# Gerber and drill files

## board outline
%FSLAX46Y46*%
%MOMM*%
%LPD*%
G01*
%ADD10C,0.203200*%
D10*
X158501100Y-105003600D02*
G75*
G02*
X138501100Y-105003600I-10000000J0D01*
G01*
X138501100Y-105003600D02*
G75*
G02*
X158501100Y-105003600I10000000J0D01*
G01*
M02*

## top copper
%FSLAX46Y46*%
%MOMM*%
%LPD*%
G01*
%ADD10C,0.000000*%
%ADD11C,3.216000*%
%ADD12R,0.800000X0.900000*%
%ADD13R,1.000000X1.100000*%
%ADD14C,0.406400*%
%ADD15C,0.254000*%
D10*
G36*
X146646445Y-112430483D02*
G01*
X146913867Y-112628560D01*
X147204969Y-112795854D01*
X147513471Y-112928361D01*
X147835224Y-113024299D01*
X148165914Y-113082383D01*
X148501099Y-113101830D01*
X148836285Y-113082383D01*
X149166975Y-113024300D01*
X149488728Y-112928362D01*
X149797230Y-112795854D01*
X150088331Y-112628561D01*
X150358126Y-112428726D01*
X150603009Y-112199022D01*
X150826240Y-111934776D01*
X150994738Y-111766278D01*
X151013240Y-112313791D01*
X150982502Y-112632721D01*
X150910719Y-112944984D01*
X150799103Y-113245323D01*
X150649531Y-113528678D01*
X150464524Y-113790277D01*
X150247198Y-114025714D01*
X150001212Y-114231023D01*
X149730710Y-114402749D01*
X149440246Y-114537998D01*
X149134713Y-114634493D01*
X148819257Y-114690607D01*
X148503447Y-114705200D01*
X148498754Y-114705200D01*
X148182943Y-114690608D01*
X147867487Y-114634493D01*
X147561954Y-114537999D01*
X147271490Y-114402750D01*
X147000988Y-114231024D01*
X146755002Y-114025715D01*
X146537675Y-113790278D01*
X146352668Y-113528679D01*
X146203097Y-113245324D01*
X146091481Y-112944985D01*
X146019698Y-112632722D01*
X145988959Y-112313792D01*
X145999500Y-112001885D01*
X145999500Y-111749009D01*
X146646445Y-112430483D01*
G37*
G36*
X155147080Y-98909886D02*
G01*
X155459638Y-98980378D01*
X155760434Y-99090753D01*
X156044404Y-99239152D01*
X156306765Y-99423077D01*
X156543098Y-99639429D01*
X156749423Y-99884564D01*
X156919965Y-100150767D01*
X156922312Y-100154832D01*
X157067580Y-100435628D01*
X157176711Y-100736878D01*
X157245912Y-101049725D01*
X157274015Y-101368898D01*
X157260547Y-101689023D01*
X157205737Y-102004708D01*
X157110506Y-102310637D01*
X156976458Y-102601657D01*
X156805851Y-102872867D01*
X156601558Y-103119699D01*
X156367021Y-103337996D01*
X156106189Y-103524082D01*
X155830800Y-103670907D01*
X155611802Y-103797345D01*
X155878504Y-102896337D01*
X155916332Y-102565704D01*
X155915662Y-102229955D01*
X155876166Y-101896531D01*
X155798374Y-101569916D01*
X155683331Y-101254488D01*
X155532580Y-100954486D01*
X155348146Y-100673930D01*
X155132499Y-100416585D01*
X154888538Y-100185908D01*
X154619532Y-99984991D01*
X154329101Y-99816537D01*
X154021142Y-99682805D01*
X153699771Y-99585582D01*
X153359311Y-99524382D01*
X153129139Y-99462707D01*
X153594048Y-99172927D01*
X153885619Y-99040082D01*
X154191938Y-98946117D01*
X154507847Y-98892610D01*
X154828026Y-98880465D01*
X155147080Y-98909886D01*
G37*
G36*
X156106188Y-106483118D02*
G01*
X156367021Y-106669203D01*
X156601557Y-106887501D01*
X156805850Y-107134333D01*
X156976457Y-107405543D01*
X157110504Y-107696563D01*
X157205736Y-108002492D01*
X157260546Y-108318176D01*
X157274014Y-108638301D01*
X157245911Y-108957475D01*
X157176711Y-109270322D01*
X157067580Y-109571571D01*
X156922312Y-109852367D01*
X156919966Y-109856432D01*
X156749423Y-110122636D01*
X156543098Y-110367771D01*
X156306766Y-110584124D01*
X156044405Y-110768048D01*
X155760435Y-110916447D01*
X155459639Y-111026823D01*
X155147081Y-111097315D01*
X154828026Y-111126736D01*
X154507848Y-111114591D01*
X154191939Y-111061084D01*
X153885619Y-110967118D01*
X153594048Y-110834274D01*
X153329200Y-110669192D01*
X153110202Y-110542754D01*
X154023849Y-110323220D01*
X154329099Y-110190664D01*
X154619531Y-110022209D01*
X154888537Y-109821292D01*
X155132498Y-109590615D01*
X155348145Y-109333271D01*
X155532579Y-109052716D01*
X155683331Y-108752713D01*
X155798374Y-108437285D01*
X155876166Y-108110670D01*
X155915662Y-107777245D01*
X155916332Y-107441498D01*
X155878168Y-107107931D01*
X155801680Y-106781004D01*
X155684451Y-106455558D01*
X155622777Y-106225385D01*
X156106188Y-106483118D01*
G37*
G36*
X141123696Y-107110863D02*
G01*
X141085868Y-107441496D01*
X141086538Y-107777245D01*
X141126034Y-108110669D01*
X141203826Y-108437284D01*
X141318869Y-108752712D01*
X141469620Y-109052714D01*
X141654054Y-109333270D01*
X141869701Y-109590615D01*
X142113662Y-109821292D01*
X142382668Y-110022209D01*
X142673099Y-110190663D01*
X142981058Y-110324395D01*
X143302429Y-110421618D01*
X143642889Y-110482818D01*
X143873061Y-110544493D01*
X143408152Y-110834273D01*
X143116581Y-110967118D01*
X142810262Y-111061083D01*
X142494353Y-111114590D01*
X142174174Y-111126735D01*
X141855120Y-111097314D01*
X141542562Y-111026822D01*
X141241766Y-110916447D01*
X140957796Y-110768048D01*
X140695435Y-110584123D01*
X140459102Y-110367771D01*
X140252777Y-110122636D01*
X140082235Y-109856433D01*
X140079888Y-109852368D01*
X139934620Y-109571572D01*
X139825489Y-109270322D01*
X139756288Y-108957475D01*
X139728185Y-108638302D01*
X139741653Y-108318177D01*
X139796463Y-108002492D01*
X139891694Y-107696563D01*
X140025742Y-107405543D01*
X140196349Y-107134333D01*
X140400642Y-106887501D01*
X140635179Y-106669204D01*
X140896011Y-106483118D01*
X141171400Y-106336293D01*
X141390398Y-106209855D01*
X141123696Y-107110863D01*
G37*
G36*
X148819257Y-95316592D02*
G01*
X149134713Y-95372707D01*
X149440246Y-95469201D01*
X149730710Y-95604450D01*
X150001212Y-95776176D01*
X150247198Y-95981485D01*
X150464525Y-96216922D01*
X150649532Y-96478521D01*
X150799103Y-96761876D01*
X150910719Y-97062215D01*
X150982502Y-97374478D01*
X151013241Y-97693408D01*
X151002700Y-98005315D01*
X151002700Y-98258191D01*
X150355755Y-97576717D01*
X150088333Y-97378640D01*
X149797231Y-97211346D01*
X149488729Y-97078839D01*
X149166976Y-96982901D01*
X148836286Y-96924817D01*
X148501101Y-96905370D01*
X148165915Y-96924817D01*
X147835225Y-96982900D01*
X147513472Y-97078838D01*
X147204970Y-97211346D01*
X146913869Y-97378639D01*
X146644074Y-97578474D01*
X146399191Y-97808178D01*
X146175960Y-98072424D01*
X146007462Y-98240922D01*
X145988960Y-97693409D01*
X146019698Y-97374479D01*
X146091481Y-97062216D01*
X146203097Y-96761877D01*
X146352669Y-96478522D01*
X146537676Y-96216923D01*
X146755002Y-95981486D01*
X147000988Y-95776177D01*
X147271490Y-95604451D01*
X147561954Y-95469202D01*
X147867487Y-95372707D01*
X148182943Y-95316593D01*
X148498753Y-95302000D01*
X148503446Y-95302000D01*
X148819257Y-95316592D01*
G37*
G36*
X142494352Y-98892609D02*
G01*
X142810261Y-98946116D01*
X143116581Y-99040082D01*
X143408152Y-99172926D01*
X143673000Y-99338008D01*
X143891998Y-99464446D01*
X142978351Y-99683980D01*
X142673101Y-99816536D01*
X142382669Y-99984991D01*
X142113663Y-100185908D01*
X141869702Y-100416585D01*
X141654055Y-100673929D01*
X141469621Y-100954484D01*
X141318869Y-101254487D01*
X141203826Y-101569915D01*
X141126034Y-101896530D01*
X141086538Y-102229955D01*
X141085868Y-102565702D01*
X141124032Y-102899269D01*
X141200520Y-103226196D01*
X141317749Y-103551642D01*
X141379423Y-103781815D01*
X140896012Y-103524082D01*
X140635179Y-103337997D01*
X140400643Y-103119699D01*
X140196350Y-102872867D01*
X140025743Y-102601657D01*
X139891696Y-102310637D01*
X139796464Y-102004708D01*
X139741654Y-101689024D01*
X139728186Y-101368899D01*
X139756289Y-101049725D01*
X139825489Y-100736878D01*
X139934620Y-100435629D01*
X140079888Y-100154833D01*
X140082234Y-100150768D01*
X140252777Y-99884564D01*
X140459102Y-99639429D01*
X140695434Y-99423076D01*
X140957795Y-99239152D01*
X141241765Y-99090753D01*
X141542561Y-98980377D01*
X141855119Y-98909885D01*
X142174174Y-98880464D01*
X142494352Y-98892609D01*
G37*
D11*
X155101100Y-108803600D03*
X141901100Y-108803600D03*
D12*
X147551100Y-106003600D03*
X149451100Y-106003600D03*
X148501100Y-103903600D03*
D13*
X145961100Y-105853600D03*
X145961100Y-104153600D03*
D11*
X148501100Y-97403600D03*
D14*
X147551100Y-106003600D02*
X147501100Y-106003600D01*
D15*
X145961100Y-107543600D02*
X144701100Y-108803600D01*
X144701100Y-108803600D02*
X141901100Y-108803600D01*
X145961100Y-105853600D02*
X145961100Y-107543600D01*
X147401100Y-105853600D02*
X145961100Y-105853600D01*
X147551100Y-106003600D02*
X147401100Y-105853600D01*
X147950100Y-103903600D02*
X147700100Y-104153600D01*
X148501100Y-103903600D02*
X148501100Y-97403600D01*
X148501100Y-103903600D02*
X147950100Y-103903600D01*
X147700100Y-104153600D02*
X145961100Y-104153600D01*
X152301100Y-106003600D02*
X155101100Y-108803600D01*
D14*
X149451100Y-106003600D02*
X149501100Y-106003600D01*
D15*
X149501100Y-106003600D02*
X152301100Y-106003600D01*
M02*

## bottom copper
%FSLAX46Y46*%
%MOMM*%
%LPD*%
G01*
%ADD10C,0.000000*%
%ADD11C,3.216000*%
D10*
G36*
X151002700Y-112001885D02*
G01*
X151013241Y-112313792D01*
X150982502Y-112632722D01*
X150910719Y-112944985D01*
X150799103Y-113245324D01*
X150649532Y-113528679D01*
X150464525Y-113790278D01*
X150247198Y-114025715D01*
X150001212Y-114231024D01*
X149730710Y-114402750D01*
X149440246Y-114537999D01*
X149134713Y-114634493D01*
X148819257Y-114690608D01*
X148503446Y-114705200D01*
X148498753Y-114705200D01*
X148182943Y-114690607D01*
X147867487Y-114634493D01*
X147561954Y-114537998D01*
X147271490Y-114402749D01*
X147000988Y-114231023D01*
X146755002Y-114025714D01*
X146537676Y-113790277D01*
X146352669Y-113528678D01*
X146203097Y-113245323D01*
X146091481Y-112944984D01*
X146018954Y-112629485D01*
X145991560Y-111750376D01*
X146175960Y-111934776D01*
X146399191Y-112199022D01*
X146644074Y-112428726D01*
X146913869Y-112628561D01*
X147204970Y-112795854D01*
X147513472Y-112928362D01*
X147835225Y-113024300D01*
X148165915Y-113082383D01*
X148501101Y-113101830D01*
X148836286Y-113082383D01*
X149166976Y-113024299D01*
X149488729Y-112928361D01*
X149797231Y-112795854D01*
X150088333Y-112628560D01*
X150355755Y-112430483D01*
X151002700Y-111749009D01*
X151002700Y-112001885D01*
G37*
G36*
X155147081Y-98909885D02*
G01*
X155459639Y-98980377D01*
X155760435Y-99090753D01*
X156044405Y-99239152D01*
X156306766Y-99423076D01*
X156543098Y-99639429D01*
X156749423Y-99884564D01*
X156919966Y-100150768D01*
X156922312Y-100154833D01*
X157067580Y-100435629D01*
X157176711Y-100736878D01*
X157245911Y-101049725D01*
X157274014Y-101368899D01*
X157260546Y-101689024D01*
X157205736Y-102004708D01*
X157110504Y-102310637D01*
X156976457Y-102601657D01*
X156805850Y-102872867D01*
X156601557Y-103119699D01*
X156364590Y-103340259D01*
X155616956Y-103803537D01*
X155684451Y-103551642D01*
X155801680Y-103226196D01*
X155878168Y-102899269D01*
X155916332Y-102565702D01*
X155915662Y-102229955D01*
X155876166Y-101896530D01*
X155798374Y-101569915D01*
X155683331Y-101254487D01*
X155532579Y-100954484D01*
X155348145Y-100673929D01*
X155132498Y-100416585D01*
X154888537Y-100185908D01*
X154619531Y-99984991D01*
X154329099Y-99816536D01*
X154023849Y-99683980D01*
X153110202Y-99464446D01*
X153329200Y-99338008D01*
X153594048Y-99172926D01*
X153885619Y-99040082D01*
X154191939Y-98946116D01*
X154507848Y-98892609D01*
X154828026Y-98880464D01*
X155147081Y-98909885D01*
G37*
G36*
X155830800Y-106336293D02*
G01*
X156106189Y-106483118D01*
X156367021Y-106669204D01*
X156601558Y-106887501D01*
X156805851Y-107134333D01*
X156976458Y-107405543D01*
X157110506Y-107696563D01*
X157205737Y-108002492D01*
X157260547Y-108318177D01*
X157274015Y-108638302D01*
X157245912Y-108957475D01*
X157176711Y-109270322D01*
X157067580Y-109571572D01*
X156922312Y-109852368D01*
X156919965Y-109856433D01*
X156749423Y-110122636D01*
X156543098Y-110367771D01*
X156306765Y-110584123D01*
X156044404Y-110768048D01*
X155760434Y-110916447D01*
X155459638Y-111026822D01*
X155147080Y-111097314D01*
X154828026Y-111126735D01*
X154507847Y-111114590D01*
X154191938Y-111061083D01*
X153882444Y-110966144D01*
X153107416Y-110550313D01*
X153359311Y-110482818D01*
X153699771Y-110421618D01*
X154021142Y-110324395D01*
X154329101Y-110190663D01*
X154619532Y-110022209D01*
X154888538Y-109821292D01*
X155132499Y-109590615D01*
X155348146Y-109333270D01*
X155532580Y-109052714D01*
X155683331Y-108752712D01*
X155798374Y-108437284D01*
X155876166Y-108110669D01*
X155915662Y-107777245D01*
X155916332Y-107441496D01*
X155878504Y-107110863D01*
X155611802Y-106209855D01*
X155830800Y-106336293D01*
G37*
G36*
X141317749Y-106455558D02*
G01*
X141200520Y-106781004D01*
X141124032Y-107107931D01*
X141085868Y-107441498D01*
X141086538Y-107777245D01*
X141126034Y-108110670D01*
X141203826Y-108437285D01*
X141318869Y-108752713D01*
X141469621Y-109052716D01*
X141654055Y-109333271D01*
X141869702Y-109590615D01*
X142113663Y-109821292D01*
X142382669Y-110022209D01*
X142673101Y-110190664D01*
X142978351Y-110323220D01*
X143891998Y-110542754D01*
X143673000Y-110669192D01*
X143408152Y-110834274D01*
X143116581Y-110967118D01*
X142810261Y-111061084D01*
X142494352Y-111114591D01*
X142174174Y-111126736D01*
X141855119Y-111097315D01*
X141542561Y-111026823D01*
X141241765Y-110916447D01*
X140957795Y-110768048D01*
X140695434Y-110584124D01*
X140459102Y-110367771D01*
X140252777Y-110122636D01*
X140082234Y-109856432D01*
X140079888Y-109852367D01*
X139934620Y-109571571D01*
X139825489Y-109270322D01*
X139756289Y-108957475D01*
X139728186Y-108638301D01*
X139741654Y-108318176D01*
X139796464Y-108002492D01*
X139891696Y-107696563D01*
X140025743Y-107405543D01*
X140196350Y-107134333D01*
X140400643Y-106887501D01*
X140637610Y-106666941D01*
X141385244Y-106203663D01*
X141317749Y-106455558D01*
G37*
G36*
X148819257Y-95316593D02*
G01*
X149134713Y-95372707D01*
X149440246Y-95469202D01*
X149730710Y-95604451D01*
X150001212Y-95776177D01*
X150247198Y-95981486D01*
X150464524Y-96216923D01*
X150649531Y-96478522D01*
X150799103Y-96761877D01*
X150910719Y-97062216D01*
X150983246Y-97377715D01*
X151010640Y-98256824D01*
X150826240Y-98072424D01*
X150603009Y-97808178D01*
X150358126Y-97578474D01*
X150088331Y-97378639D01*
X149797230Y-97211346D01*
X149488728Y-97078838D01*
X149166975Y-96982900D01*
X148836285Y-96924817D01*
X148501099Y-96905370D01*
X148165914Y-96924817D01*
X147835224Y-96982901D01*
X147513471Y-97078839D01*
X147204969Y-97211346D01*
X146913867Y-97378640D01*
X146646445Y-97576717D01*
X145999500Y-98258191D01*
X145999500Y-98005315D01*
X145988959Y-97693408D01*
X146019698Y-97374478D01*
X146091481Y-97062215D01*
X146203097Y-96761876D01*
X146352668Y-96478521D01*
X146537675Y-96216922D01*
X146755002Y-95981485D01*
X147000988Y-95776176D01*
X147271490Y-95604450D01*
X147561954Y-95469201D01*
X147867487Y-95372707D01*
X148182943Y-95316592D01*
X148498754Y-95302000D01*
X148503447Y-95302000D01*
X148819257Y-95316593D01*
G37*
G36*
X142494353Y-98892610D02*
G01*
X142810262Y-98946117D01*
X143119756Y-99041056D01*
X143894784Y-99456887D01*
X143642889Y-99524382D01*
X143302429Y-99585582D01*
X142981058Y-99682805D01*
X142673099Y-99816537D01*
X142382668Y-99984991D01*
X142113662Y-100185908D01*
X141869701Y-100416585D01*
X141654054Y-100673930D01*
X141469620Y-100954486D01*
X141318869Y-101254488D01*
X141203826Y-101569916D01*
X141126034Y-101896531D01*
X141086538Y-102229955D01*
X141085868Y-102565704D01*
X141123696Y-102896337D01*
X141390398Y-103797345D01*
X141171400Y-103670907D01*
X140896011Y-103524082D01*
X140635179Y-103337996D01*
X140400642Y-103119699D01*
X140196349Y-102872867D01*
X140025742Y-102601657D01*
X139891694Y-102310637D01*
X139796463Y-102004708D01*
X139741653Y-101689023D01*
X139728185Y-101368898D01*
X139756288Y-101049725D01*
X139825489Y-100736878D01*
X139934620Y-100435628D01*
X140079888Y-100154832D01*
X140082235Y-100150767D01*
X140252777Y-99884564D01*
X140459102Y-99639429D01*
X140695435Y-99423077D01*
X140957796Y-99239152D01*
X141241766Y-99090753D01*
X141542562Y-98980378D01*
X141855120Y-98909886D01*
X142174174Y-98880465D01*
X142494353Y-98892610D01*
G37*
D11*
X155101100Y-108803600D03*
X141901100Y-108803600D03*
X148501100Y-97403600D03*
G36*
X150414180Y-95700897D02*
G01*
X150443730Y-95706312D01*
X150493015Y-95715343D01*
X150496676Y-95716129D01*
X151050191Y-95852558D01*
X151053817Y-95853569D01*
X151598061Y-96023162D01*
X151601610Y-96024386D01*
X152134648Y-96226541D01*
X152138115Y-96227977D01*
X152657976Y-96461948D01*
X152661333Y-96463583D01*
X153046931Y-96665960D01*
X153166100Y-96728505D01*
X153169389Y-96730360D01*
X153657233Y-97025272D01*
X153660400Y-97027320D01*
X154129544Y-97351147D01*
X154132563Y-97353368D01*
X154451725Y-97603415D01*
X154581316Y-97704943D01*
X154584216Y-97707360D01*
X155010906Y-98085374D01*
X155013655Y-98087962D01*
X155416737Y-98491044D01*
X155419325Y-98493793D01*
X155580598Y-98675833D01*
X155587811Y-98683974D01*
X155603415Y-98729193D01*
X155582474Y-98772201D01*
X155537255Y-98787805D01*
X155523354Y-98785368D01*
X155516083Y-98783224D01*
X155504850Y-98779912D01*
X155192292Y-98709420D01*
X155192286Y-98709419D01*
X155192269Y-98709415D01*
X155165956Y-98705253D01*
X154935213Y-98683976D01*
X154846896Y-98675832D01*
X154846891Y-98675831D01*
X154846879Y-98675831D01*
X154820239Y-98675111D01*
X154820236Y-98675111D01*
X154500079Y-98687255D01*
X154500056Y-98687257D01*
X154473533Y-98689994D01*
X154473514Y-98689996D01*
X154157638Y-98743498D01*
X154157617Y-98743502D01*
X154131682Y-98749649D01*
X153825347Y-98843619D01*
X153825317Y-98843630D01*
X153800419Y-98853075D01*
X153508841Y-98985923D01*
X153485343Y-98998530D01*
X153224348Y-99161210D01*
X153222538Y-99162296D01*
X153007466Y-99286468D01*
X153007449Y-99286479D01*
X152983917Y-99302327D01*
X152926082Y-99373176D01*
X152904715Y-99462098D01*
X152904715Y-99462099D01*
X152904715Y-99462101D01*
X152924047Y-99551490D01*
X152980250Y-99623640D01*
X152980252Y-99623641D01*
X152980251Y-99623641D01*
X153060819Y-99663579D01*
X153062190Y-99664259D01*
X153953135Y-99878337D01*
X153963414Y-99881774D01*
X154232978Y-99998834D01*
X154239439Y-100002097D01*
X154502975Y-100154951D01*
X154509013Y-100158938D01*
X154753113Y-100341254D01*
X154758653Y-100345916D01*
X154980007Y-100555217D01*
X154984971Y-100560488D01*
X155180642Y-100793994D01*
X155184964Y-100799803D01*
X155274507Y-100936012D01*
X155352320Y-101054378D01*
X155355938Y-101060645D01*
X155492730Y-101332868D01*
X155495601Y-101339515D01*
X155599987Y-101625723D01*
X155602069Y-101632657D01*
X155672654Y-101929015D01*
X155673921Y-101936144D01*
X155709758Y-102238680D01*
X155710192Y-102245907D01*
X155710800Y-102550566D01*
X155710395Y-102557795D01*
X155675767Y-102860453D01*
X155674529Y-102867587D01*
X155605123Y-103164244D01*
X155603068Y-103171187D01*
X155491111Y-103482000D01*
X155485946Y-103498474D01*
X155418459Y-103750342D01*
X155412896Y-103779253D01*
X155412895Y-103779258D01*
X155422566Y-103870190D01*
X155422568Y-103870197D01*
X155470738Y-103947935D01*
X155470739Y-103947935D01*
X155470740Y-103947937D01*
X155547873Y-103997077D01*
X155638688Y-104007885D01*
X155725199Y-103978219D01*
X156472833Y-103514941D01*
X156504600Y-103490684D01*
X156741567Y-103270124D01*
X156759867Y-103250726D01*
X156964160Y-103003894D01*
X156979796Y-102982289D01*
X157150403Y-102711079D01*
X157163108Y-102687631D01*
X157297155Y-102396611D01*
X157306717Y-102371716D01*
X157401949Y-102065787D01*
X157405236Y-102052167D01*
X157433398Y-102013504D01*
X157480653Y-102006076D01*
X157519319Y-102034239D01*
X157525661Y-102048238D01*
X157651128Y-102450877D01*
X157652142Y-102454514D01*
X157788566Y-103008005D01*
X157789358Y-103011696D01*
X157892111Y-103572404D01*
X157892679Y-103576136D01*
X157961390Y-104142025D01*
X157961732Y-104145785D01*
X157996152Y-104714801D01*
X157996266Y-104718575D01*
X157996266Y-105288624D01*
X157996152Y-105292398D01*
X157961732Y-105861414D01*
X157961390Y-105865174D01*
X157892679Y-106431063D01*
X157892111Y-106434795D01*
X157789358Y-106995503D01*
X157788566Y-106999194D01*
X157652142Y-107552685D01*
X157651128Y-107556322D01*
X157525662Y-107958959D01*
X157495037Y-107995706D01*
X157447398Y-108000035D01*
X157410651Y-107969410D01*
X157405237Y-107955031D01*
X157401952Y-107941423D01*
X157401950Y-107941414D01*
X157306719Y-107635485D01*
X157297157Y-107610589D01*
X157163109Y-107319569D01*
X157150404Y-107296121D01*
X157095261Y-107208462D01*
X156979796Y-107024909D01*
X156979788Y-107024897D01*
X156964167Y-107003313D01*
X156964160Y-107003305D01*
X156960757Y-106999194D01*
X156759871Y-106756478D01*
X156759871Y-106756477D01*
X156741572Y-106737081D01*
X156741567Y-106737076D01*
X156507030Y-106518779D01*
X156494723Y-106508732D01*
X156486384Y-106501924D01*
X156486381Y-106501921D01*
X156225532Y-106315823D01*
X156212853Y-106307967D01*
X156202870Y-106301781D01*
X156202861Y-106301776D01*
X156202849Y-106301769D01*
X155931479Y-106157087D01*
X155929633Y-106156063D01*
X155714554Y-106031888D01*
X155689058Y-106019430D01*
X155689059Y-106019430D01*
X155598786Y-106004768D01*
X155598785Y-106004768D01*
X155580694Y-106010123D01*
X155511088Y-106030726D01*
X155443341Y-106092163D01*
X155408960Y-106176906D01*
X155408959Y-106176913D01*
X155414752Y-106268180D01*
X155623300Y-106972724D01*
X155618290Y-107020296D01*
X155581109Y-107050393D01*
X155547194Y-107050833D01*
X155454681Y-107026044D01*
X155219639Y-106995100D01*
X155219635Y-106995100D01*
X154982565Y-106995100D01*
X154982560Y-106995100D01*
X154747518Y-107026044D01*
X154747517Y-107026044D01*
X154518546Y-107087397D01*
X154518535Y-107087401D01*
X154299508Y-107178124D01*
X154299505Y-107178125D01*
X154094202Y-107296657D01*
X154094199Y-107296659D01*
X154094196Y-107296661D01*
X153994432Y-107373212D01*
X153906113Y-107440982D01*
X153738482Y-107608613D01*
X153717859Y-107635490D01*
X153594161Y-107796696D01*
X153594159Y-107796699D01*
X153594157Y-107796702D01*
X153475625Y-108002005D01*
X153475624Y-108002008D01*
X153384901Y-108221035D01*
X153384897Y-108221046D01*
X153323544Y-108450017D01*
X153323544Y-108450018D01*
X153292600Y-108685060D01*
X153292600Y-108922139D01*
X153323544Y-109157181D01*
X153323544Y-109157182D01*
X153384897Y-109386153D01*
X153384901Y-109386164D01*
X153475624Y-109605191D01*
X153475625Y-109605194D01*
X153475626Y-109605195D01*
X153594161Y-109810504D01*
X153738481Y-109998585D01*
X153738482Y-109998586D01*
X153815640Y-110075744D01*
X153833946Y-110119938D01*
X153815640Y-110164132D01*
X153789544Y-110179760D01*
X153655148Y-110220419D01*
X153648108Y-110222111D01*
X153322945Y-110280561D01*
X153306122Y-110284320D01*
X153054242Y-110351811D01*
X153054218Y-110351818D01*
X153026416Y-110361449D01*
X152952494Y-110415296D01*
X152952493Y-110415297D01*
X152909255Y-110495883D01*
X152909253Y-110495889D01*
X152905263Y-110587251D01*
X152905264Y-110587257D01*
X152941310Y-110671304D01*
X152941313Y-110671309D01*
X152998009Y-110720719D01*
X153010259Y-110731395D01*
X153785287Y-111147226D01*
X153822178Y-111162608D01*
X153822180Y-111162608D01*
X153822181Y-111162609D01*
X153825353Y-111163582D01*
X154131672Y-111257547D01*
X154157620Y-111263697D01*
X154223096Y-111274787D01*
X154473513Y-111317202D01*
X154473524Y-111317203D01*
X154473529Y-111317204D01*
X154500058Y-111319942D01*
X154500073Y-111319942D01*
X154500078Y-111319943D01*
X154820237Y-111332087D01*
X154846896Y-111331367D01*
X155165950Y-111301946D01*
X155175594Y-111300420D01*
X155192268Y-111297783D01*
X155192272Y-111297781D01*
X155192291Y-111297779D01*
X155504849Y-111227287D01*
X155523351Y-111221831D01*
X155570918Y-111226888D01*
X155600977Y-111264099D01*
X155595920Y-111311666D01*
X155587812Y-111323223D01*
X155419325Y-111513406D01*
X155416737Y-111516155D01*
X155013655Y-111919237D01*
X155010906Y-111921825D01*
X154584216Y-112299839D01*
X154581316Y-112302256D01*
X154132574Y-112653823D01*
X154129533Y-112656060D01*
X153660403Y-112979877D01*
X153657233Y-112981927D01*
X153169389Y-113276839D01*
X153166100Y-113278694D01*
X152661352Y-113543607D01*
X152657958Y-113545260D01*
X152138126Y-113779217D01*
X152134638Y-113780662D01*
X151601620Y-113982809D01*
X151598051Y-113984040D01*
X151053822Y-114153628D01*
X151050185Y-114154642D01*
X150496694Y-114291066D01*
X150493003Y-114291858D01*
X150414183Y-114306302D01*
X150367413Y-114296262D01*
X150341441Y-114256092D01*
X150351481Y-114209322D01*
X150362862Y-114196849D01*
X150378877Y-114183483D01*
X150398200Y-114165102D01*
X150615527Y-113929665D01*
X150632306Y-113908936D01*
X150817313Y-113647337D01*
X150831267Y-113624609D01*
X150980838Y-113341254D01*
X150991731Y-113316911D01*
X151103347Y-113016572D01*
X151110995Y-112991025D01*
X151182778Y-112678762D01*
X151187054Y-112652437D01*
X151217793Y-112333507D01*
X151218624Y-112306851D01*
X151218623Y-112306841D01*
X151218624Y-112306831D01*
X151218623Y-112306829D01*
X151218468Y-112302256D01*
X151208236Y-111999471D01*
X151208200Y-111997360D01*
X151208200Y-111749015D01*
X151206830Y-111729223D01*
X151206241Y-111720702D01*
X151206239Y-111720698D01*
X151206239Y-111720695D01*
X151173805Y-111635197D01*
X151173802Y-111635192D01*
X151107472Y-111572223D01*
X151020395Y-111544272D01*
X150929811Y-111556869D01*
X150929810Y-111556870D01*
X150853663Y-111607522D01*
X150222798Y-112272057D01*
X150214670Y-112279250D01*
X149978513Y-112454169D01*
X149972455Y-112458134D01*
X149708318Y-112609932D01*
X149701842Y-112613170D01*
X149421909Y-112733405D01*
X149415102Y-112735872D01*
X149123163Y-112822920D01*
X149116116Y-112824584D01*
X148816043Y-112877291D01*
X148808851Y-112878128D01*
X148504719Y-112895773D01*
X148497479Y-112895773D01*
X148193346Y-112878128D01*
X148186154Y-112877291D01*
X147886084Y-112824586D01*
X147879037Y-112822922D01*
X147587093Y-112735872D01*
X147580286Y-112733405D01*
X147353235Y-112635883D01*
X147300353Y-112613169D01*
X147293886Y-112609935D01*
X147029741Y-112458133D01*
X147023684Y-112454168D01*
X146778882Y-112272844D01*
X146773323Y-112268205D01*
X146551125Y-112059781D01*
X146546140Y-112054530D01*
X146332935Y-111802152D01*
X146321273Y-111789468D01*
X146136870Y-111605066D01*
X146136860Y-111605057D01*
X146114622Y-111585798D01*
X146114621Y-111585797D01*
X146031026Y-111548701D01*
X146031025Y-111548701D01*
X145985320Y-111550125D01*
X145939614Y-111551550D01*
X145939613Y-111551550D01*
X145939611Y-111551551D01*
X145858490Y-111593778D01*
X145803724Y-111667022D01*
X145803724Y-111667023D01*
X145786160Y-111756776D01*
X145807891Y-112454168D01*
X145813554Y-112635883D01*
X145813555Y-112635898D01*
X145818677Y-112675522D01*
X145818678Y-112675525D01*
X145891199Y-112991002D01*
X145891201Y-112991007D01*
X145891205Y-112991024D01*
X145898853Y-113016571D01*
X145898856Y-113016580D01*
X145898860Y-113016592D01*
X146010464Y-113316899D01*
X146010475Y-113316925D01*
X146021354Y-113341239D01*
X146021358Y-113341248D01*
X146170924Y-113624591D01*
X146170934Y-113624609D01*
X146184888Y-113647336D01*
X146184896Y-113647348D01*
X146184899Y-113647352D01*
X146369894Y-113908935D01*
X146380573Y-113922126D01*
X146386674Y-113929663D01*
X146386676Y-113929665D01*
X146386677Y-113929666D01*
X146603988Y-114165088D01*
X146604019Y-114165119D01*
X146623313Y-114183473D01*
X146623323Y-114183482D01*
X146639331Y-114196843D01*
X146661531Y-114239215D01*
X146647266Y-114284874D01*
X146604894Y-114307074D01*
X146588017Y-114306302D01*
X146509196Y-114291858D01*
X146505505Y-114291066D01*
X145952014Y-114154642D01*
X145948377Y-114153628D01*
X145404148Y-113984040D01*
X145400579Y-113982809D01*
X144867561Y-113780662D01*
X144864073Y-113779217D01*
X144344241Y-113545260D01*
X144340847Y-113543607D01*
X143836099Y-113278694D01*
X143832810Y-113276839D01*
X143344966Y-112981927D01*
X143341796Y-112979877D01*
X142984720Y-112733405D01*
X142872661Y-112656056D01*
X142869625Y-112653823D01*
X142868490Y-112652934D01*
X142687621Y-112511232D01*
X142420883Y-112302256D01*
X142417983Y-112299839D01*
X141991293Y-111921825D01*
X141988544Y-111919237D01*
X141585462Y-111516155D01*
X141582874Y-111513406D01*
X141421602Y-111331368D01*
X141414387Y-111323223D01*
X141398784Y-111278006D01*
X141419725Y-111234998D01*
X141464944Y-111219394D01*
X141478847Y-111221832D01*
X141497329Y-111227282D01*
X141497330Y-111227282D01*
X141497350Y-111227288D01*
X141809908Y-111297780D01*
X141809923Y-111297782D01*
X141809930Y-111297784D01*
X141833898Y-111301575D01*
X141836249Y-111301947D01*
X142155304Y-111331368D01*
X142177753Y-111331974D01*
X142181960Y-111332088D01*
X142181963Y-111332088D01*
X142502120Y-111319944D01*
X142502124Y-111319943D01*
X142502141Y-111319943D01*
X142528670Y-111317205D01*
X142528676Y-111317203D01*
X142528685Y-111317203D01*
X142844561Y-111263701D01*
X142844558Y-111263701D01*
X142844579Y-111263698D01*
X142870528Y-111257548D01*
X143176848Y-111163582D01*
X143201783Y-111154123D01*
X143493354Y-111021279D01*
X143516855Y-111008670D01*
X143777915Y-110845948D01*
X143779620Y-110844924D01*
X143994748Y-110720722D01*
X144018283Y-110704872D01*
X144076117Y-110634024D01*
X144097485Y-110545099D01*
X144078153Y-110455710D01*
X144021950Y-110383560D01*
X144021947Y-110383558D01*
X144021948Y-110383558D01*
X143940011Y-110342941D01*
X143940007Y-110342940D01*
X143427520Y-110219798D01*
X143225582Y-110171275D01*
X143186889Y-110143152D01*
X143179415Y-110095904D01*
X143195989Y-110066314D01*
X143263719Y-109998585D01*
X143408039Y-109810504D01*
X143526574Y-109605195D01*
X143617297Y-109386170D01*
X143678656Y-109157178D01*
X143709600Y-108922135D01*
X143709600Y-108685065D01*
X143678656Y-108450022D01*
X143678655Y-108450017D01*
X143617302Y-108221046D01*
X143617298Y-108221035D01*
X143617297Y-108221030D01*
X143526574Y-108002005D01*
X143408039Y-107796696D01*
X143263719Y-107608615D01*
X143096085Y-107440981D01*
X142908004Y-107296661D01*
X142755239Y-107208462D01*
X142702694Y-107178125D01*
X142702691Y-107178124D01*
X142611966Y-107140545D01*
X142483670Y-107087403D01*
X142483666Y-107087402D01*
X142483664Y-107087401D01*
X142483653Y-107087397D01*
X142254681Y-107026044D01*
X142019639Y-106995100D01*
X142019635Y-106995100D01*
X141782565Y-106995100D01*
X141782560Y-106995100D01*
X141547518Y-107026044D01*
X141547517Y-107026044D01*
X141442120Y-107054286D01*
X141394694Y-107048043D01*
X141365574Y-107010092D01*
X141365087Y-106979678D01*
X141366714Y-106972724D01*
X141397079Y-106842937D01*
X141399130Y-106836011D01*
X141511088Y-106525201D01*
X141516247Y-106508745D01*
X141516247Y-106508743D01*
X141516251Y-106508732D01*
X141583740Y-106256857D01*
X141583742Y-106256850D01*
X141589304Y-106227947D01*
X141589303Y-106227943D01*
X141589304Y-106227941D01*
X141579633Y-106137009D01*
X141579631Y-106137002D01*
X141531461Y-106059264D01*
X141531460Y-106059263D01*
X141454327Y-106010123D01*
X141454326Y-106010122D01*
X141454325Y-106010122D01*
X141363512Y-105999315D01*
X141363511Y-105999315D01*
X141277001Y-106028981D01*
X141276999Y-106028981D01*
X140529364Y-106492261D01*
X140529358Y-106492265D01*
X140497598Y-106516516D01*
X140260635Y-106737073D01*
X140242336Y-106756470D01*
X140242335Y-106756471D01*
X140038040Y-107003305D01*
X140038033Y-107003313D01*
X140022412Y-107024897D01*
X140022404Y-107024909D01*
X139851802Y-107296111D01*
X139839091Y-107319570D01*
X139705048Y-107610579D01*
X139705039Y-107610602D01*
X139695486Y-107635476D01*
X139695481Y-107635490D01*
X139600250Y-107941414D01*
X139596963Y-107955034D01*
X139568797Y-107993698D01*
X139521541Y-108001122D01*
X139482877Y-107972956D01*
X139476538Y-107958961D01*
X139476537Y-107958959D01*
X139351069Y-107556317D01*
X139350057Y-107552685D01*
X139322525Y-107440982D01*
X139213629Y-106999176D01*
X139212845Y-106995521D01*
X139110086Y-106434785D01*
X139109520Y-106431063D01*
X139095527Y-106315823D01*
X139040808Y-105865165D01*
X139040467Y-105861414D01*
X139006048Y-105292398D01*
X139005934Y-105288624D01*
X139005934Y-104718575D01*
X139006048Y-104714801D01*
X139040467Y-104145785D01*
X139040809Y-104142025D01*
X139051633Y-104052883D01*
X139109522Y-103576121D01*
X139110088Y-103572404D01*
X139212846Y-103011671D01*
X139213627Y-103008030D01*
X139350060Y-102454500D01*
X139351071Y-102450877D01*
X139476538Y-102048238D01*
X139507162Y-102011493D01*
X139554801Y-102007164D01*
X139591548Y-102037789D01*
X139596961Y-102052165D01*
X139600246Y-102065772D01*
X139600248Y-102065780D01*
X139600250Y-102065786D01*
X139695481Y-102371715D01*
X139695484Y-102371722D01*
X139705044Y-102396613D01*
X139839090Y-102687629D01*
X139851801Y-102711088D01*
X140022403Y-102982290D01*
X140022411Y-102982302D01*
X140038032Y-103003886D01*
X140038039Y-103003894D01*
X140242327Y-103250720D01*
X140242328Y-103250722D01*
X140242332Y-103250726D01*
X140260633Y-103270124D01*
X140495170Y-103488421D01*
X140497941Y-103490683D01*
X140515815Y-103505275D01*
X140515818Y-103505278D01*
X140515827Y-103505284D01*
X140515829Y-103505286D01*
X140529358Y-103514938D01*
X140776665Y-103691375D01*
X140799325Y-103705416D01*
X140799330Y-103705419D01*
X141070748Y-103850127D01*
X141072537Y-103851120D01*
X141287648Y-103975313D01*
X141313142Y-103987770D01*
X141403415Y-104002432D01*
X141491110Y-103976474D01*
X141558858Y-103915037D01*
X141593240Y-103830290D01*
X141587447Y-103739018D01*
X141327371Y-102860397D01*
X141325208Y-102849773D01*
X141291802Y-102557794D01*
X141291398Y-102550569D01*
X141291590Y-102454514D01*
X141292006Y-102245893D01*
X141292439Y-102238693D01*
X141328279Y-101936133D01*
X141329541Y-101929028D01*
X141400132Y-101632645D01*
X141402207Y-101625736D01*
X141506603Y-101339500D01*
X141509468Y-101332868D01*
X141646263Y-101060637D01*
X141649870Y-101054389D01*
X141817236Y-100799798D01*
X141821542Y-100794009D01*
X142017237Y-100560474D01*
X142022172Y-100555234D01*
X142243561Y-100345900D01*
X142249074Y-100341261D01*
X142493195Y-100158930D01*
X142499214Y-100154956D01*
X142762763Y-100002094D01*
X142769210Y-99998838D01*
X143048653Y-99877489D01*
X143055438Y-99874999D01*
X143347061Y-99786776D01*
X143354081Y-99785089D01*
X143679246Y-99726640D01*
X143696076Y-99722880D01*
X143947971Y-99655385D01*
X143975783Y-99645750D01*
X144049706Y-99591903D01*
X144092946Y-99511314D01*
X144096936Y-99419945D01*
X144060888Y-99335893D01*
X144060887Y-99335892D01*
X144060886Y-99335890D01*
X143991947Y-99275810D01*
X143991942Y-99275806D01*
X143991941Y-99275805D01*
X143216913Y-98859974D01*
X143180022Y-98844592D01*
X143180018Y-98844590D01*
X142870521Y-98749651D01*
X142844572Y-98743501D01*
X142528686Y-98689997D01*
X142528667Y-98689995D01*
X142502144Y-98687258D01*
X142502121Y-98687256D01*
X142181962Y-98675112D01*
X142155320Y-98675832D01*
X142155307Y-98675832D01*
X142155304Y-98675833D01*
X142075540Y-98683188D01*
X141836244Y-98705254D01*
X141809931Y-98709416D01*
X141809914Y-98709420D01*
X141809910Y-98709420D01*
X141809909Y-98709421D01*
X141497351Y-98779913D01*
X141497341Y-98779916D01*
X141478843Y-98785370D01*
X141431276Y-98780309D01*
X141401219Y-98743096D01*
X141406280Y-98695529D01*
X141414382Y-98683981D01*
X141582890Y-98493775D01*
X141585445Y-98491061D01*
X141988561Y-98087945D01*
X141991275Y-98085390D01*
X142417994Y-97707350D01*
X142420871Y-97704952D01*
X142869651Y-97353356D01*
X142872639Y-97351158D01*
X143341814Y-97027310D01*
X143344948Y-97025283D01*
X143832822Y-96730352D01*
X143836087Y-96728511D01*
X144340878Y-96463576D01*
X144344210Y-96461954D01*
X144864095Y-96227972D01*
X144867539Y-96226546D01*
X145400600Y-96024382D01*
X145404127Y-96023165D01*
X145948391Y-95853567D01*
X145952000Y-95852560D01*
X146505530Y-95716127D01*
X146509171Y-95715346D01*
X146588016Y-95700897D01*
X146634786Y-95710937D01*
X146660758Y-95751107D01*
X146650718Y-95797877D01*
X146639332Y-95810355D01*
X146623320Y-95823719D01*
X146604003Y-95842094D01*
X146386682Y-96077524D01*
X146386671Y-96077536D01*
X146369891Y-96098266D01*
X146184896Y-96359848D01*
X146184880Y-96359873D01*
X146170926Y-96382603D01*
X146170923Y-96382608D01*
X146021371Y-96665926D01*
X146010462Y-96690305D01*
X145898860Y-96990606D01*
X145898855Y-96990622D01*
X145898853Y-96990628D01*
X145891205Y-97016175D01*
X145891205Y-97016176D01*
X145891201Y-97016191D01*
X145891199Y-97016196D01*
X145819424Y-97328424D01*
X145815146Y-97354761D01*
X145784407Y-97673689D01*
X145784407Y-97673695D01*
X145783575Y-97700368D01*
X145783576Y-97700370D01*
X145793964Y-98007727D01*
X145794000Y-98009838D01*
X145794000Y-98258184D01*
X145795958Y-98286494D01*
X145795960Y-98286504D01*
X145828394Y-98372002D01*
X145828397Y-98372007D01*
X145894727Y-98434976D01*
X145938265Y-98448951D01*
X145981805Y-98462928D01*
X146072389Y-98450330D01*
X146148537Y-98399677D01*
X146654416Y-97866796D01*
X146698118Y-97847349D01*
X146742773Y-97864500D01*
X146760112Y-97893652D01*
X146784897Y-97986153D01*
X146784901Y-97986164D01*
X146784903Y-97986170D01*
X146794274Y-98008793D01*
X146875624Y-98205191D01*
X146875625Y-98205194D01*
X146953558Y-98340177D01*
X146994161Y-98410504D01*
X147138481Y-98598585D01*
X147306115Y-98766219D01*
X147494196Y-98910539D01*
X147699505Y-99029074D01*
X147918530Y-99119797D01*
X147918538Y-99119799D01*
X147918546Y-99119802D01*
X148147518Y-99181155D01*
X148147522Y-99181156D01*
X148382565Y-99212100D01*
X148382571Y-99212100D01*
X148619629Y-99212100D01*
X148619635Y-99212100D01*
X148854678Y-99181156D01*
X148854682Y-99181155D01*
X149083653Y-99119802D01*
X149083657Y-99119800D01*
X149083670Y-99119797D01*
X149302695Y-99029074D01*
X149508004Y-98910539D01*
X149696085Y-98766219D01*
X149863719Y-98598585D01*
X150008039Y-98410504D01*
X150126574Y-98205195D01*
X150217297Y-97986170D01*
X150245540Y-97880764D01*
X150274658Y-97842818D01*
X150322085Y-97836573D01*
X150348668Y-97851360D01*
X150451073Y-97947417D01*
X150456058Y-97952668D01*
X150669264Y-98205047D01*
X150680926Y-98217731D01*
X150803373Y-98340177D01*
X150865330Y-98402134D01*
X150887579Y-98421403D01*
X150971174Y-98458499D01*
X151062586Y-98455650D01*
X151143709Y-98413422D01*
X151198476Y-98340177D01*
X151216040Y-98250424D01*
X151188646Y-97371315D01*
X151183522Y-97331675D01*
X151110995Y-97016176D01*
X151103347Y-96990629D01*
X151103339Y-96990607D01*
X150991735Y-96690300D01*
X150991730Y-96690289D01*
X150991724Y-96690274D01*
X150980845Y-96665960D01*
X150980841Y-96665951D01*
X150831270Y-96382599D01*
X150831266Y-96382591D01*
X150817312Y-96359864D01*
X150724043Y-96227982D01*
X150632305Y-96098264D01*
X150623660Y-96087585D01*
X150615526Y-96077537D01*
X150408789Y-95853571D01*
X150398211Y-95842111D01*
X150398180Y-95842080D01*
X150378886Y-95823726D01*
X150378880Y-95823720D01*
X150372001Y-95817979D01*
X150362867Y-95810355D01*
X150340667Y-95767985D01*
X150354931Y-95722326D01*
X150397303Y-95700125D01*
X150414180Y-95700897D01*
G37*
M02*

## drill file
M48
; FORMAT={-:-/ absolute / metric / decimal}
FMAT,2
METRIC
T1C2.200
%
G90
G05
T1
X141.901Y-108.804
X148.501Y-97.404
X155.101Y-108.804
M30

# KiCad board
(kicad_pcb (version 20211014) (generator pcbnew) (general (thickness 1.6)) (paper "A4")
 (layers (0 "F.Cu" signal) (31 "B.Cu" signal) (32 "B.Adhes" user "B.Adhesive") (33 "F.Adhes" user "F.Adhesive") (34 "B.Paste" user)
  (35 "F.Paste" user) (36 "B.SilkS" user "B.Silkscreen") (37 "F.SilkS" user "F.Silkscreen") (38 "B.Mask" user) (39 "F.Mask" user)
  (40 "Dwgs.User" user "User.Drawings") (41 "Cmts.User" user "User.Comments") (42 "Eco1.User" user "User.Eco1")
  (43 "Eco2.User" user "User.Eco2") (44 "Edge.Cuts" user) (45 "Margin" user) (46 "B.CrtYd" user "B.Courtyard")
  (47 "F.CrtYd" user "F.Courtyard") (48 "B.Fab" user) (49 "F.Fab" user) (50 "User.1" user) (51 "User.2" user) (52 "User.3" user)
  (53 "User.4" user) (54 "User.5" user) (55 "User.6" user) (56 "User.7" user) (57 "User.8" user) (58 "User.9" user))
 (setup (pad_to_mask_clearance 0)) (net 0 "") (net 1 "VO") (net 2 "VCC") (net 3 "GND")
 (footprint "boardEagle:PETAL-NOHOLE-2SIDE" (layer "F.Cu") (at 148.5011 112.6036)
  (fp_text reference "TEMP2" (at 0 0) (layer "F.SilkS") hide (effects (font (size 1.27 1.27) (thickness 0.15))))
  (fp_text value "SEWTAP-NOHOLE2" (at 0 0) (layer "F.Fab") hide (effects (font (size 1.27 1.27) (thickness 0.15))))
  (fp_poly
   (pts (xy -1.854655 -0.173117) (xy -1.587233 0.02496) (xy -1.296131 0.192254) (xy -0.987629 0.324761) (xy -0.665876 0.420699)
    (xy -0.335186 0.478783) (xy -0.000001 0.49823) (xy 0.335185 0.478783) (xy 0.665875 0.4207) (xy 0.987628 0.324762) (xy 1.29613 0.192254)
    (xy 1.587231 0.024961) (xy 1.857026 -0.174874) (xy 2.101909 -0.404578) (xy 2.32514 -0.668824) (xy 2.493638 -0.837322)
    (xy 2.51214 -0.289809) (xy 2.481402 0.029121) (xy 2.409619 0.341384) (xy 2.298003 0.641723) (xy 2.148431 0.925078)
    (xy 1.963424 1.186677) (xy 1.746098 1.422114) (xy 1.500112 1.627423) (xy 1.22961 1.799149) (xy 0.939146 1.934398) (xy 0.633613 2.030893)
    (xy 0.318157 2.087007) (xy 0.002347 2.1016) (xy -0.002346 2.1016) (xy -0.318157 2.087008) (xy -0.633613 2.030893)
    (xy -0.939146 1.934399) (xy -1.22961 1.79915) (xy -1.500112 1.627424) (xy -1.746098 1.422115) (xy -1.963425 1.186678)
    (xy -2.148432 0.925079) (xy -2.298003 0.641724) (xy -2.409619 0.341385) (xy -2.481402 0.029122) (xy -2.512141 -0.289808)
    (xy -2.5016 -0.601715) (xy -2.5016 -0.854591))
   (layer "F.Cu") (width 0) (fill solid))
  (fp_poly
   (pts (xy 2.5016 -0.601715) (xy 2.512141 -0.289808) (xy 2.481402 0.029122) (xy 2.409619 0.341385) (xy 2.298003 0.641724)
    (xy 2.148432 0.925079) (xy 1.963425 1.186678) (xy 1.746098 1.422115) (xy 1.500112 1.627424) (xy 1.22961 1.79915) (xy 0.939146 1.934399)
    (xy 0.633613 2.030893) (xy 0.318157 2.087008) (xy 0.002346 2.1016) (xy -0.002347 2.1016) (xy -0.318157 2.087007) (xy -0.633613 2.030893)
    (xy -0.939146 1.934398) (xy -1.22961 1.799149) (xy -1.500112 1.627423) (xy -1.746098 1.422114) (xy -1.963424 1.186677)
    (xy -2.148431 0.925078) (xy -2.298003 0.641723) (xy -2.409619 0.341384) (xy -2.482146 0.025885) (xy -2.50954 -0.853224)
    (xy -2.32514 -0.668824) (xy -2.101909 -0.404578) (xy -1.857026 -0.174874) (xy -1.587231 0.024961) (xy -1.29613 0.192254)
    (xy -0.987628 0.324762) (xy -0.665875 0.4207) (xy -0.335185 0.478783) (xy 0.000001 0.49823) (xy 0.335186 0.478783)
    (xy 0.665876 0.420699) (xy 0.987629 0.324761) (xy 1.296131 0.192254) (xy 1.587233 0.02496) (xy 1.854655 -0.173117) (xy 2.5016 -0.854591))
   (layer "B.Cu") (width 0) (fill solid)))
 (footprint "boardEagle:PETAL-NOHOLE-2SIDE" (layer "F.Cu") (at 155.1011 101.2036 120)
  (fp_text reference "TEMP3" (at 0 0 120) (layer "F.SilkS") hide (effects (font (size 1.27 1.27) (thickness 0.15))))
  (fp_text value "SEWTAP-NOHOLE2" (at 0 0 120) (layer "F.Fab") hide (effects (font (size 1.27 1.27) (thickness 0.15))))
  (fp_poly
   (pts (xy -1.854655 -0.173117) (xy -1.587233 0.02496) (xy -1.296131 0.192254) (xy -0.987629 0.324761) (xy -0.665876 0.420699)
    (xy -0.335186 0.478783) (xy -0.000001 0.49823) (xy 0.335185 0.478783) (xy 0.665875 0.4207) (xy 0.987628 0.324762) (xy 1.29613 0.192254)
    (xy 1.587231 0.024961) (xy 1.857026 -0.174874) (xy 2.101909 -0.404578) (xy 2.32514 -0.668824) (xy 2.493638 -0.837322)
    (xy 2.51214 -0.289809) (xy 2.481402 0.029121) (xy 2.409619 0.341384) (xy 2.298003 0.641723) (xy 2.148431 0.925078)
    (xy 1.963424 1.186677) (xy 1.746098 1.422114) (xy 1.500112 1.627423) (xy 1.22961 1.799149) (xy 0.939146 1.934398) (xy 0.633613 2.030893)
    (xy 0.318157 2.087007) (xy 0.002347 2.1016) (xy -0.002346 2.1016) (xy -0.318157 2.087008) (xy -0.633613 2.030893)
    (xy -0.939146 1.934399) (xy -1.22961 1.79915) (xy -1.500112 1.627424) (xy -1.746098 1.422115) (xy -1.963425 1.186678)
    (xy -2.148432 0.925079) (xy -2.298003 0.641724) (xy -2.409619 0.341385) (xy -2.481402 0.029122) (xy -2.512141 -0.289808)
    (xy -2.5016 -0.601715) (xy -2.5016 -0.854591))
   (layer "F.Cu") (width 0) (fill solid))
  (fp_poly
   (pts (xy 2.5016 -0.601715) (xy 2.512141 -0.289808) (xy 2.481402 0.029122) (xy 2.409619 0.341385) (xy 2.298003 0.641724)
    (xy 2.148432 0.925079) (xy 1.963425 1.186678) (xy 1.746098 1.422115) (xy 1.500112 1.627424) (xy 1.22961 1.79915) (xy 0.939146 1.934399)
    (xy 0.633613 2.030893) (xy 0.318157 2.087008) (xy 0.002346 2.1016) (xy -0.002347 2.1016) (xy -0.318157 2.087007) (xy -0.633613 2.030893)
    (xy -0.939146 1.934398) (xy -1.22961 1.799149) (xy -1.500112 1.627423) (xy -1.746098 1.422114) (xy -1.963424 1.186677)
    (xy -2.148431 0.925078) (xy -2.298003 0.641723) (xy -2.409619 0.341384) (xy -2.482146 0.025885) (xy -2.50954 -0.853224)
    (xy -2.32514 -0.668824) (xy -2.101909 -0.404578) (xy -1.857026 -0.174874) (xy -1.587231 0.024961) (xy -1.29613 0.192254)
    (xy -0.987628 0.324762) (xy -0.665875 0.4207) (xy -0.335185 0.478783) (xy 0.000001 0.49823) (xy 0.335186 0.478783)
    (xy 0.665876 0.420699) (xy 0.987629 0.324761) (xy 1.296131 0.192254) (xy 1.587233 0.02496) (xy 1.854655 -0.173117) (xy 2.5016 -0.854591))
   (layer "B.Cu") (width 0) (fill solid)))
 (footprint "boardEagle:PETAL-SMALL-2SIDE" (layer "F.Cu") (at 155.1011 108.8036 60)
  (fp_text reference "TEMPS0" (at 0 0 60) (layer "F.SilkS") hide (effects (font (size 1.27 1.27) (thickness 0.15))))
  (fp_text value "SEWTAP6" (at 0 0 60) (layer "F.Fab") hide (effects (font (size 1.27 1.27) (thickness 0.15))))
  (fp_poly
   (pts (xy -1.854655 -0.173117) (xy -1.587233 0.02496) (xy -1.296131 0.192254) (xy -0.987629 0.324761) (xy -0.665876 0.420699)
    (xy -0.335186 0.478783) (xy -0.000001 0.49823) (xy 0.335185 0.478783) (xy 0.665875 0.4207) (xy 0.987628 0.324762) (xy 1.29613 0.192254)
    (xy 1.587231 0.024961) (xy 1.857026 -0.174874) (xy 2.101909 -0.404578) (xy 2.32514 -0.668824) (xy 2.493638 -0.837322)
    (xy 2.51214 -0.289809) (xy 2.481402 0.029121) (xy 2.409619 0.341384) (xy 2.298003 0.641723) (xy 2.148431 0.925078)
    (xy 1.963424 1.186677) (xy 1.746098 1.422114) (xy 1.500112 1.627423) (xy 1.22961 1.799149) (xy 0.939146 1.934398) (xy 0.633613 2.030893)
    (xy 0.318157 2.087007) (xy 0.002347 2.1016) (xy -0.002346 2.1016) (xy -0.318157 2.087008) (xy -0.633613 2.030893)
    (xy -0.939146 1.934399) (xy -1.22961 1.79915) (xy -1.500112 1.627424) (xy -1.746098 1.422115) (xy -1.963425 1.186678)
    (xy -2.148432 0.925079) (xy -2.298003 0.641724) (xy -2.409619 0.341385) (xy -2.481402 0.029122) (xy -2.512141 -0.289808)
    (xy -2.5016 -0.601715) (xy -2.5016 -0.854591))
   (layer "F.Cu") (width 0) (fill solid))
  (fp_poly
   (pts (xy 2.5016 -0.601715) (xy 2.512141 -0.289808) (xy 2.481402 0.029122) (xy 2.409619 0.341385) (xy 2.298003 0.641724)
    (xy 2.148432 0.925079) (xy 1.963425 1.186678) (xy 1.746098 1.422115) (xy 1.500112 1.627424) (xy 1.22961 1.79915) (xy 0.939146 1.934399)
    (xy 0.633613 2.030893) (xy 0.318157 2.087008) (xy 0.002346 2.1016) (xy -0.002347 2.1016) (xy -0.318157 2.087007) (xy -0.633613 2.030893)
    (xy -0.939146 1.934398) (xy -1.22961 1.799149) (xy -1.500112 1.627423) (xy -1.746098 1.422114) (xy -1.963424 1.186677)
    (xy -2.148431 0.925078) (xy -2.298003 0.641723) (xy -2.409619 0.341384) (xy -2.482146 0.025885) (xy -2.50954 -0.853224)
    (xy -2.32514 -0.668824) (xy -2.101909 -0.404578) (xy -1.857026 -0.174874) (xy -1.587231 0.024961) (xy -1.29613 0.192254)
    (xy -0.987628 0.324762) (xy -0.665875 0.4207) (xy -0.335185 0.478783) (xy 0.000001 0.49823) (xy 0.335186 0.478783)
    (xy 0.665876 0.420699) (xy 0.987629 0.324761) (xy 1.296131 0.192254) (xy 1.587233 0.02496) (xy 1.854655 -0.173117) (xy 2.5016 -0.854591))
   (layer "B.Cu") (width 0) (fill solid))
  (pad "1" thru_hole circle (at 0 0 150) (size 3.216 3.216) (drill 2.2) (layers *.Cu *.Mask) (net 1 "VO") (solder_mask_margin 0.1016)))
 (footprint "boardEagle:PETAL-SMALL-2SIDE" (layer "F.Cu") (at 141.9011 108.8036 -60)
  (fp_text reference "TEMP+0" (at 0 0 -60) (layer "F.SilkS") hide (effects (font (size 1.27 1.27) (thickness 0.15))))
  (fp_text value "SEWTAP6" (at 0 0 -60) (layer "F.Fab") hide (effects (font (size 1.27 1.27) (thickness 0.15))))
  (fp_poly
   (pts (xy -1.854655 -0.173117) (xy -1.587233 0.02496) (xy -1.296131 0.192254) (xy -0.987629 0.324761) (xy -0.665876 0.420699)
    (xy -0.335186 0.478783) (xy -0.000001 0.49823) (xy 0.335185 0.478783) (xy 0.665875 0.4207) (xy 0.987628 0.324762) (xy 1.29613 0.192254)
    (xy 1.587231 0.024961) (xy 1.857026 -0.174874) (xy 2.101909 -0.404578) (xy 2.32514 -0.668824) (xy 2.493638 -0.837322)
    (xy 2.51214 -0.289809) (xy 2.481402 0.029121) (xy 2.409619 0.341384) (xy 2.298003 0.641723) (xy 2.148431 0.925078)
    (xy 1.963424 1.186677) (xy 1.746098 1.422114) (xy 1.500112 1.627423) (xy 1.22961 1.799149) (xy 0.939146 1.934398) (xy 0.633613 2.030893)
    (xy 0.318157 2.087007) (xy 0.002347 2.1016) (xy -0.002346 2.1016) (xy -0.318157 2.087008) (xy -0.633613 2.030893)
    (xy -0.939146 1.934399) (xy -1.22961 1.79915) (xy -1.500112 1.627424) (xy -1.746098 1.422115) (xy -1.963425 1.186678)
    (xy -2.148432 0.925079) (xy -2.298003 0.641724) (xy -2.409619 0.341385) (xy -2.481402 0.029122) (xy -2.512141 -0.289808)
    (xy -2.5016 -0.601715) (xy -2.5016 -0.854591))
   (layer "F.Cu") (width 0) (fill solid))
  (fp_poly
   (pts (xy 2.5016 -0.601715) (xy 2.512141 -0.289808) (xy 2.481402 0.029122) (xy 2.409619 0.341385) (xy 2.298003 0.641724)
    (xy 2.148432 0.925079) (xy 1.963425 1.186678) (xy 1.746098 1.422115) (xy 1.500112 1.627424) (xy 1.22961 1.79915) (xy 0.939146 1.934399)
    (xy 0.633613 2.030893) (xy 0.318157 2.087008) (xy 0.002346 2.1016) (xy -0.002347 2.1016) (xy -0.318157 2.087007) (xy -0.633613 2.030893)
    (xy -0.939146 1.934398) (xy -1.22961 1.799149) (xy -1.500112 1.627423) (xy -1.746098 1.422114) (xy -1.963424 1.186677)
    (xy -2.148431 0.925078) (xy -2.298003 0.641723) (xy -2.409619 0.341384) (xy -2.482146 0.025885) (xy -2.50954 -0.853224)
    (xy -2.32514 -0.668824) (xy -2.101909 -0.404578) (xy -1.857026 -0.174874) (xy -1.587231 0.024961) (xy -1.29613 0.192254)
    (xy -0.987628 0.324762) (xy -0.665875 0.4207) (xy -0.335185 0.478783) (xy 0.000001 0.49823) (xy 0.335186 0.478783)
    (xy 0.665876 0.420699) (xy 0.987629 0.324761) (xy 1.296131 0.192254) (xy 1.587233 0.02496) (xy 1.854655 -0.173117) (xy 2.5016 -0.854591))
   (layer "B.Cu") (width 0) (fill solid))
  (pad "1" thru_hole circle (at 0 0 30) (size 3.216 3.216) (drill 2.2) (layers *.Cu *.Mask) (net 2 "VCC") (solder_mask_margin 0.1016)))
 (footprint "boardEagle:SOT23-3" (layer "F.Cu") (at 148.5011 105.0036)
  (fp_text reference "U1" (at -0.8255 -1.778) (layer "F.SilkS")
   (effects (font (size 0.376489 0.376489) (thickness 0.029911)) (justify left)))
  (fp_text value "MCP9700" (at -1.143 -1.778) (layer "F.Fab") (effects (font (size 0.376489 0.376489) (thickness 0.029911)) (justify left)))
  (pad "1" smd rect (at -0.95 1) (size 0.8 0.9) (layers "F.Cu" "F.Paste" "F.Mask") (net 2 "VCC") (solder_mask_margin 0.1016))
  (pad "2" smd rect (at 0.95 1) (size 0.8 0.9) (layers "F.Cu" "F.Paste" "F.Mask") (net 1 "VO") (solder_mask_margin 0.1016))
  (pad "3" smd rect (at 0 -1.1) (size 0.8 0.9) (layers "F.Cu" "F.Paste" "F.Mask") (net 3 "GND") (solder_mask_margin 0.1016)))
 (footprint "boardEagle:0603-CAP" (layer "F.Cu") (at 145.9611 105.0036 90)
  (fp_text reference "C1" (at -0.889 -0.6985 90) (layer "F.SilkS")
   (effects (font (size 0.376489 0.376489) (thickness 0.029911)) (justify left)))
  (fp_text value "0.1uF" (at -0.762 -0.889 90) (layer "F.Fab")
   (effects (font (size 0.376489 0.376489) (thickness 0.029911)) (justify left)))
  (pad "1" smd rect (at -0.85 0 90) (size 1.1 1) (layers "F.Cu" "F.Paste" "F.Mask") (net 2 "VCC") (solder_mask_margin 0.1016))
  (pad "2" smd rect (at 0.85 0 90) (size 1.1 1) (layers "F.Cu" "F.Paste" "F.Mask") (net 3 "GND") (solder_mask_margin 0.1016)))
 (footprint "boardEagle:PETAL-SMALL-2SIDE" (layer "F.Cu") (at 148.5011 97.4036 180)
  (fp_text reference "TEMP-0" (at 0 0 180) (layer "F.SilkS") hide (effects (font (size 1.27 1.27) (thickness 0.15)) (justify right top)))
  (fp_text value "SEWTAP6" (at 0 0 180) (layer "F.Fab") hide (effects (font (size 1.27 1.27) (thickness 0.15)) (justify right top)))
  (fp_poly
   (pts (xy -1.854655 -0.173117) (xy -1.587233 0.02496) (xy -1.296131 0.192254) (xy -0.987629 0.324761) (xy -0.665876 0.420699)
    (xy -0.335186 0.478783) (xy -0.000001 0.49823) (xy 0.335185 0.478783) (xy 0.665875 0.4207) (xy 0.987628 0.324762) (xy 1.29613 0.192254)
    (xy 1.587231 0.024961) (xy 1.857026 -0.174874) (xy 2.101909 -0.404578) (xy 2.32514 -0.668824) (xy 2.493638 -0.837322)
    (xy 2.51214 -0.289809) (xy 2.481402 0.029121) (xy 2.409619 0.341384) (xy 2.298003 0.641723) (xy 2.148431 0.925078)
    (xy 1.963424 1.186677) (xy 1.746098 1.422114) (xy 1.500112 1.627423) (xy 1.22961 1.799149) (xy 0.939146 1.934398) (xy 0.633613 2.030893)
    (xy 0.318157 2.087007) (xy 0.002347 2.1016) (xy -0.002346 2.1016) (xy -0.318157 2.087008) (xy -0.633613 2.030893)
    (xy -0.939146 1.934399) (xy -1.22961 1.79915) (xy -1.500112 1.627424) (xy -1.746098 1.422115) (xy -1.963425 1.186678)
    (xy -2.148432 0.925079) (xy -2.298003 0.641724) (xy -2.409619 0.341385) (xy -2.481402 0.029122) (xy -2.512141 -0.289808)
    (xy -2.5016 -0.601715) (xy -2.5016 -0.854591))
   (layer "F.Cu") (width 0) (fill solid))
  (fp_poly
   (pts (xy 2.5016 -0.601715) (xy 2.512141 -0.289808) (xy 2.481402 0.029122) (xy 2.409619 0.341385) (xy 2.298003 0.641724)
    (xy 2.148432 0.925079) (xy 1.963425 1.186678) (xy 1.746098 1.422115) (xy 1.500112 1.627424) (xy 1.22961 1.79915) (xy 0.939146 1.934399)
    (xy 0.633613 2.030893) (xy 0.318157 2.087008) (xy 0.002346 2.1016) (xy -0.002347 2.1016) (xy -0.318157 2.087007) (xy -0.633613 2.030893)
    (xy -0.939146 1.934398) (xy -1.22961 1.799149) (xy -1.500112 1.627423) (xy -1.746098 1.422114) (xy -1.963424 1.186677)
    (xy -2.148431 0.925078) (xy -2.298003 0.641723) (xy -2.409619 0.341384) (xy -2.482146 0.025885) (xy -2.50954 -0.853224)
    (xy -2.32514 -0.668824) (xy -2.101909 -0.404578) (xy -1.857026 -0.174874) (xy -1.587231 0.024961) (xy -1.29613 0.192254)
    (xy -0.987628 0.324762) (xy -0.665875 0.4207) (xy -0.335185 0.478783) (xy 0.000001 0.49823) (xy 0.335186 0.478783)
    (xy 0.665876 0.420699) (xy 0.987629 0.324761) (xy 1.296131 0.192254) (xy 1.587233 0.02496) (xy 1.854655 -0.173117) (xy 2.5016 -0.854591))
   (layer "B.Cu") (width 0) (fill solid))
  (pad "1" thru_hole circle (at 0 0 270) (size 3.216 3.216) (drill 2.2) (layers *.Cu *.Mask) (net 3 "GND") (solder_mask_margin 0.1016)))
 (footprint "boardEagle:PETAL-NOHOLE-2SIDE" (layer "F.Cu") (at 141.9011 101.2036 -120)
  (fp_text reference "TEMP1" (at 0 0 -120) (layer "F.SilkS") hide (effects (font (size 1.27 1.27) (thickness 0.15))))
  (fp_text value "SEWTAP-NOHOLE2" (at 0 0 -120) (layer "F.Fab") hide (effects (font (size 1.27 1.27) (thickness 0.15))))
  (fp_poly
   (pts (xy -1.854655 -0.173117) (xy -1.587233 0.02496) (xy -1.296131 0.192254) (xy -0.987629 0.324761) (xy -0.665876 0.420699)
    (xy -0.335186 0.478783) (xy -0.000001 0.49823) (xy 0.335185 0.478783) (xy 0.665875 0.4207) (xy 0.987628 0.324762) (xy 1.29613 0.192254)
    (xy 1.587231 0.024961) (xy 1.857026 -0.174874) (xy 2.101909 -0.404578) (xy 2.32514 -0.668824) (xy 2.493638 -0.837322)
    (xy 2.51214 -0.289809) (xy 2.481402 0.029121) (xy 2.409619 0.341384) (xy 2.298003 0.641723) (xy 2.148431 0.925078)
    (xy 1.963424 1.186677) (xy 1.746098 1.422114) (xy 1.500112 1.627423) (xy 1.22961 1.799149) (xy 0.939146 1.934398) (xy 0.633613 2.030893)
    (xy 0.318157 2.087007) (xy 0.002347 2.1016) (xy -0.002346 2.1016) (xy -0.318157 2.087008) (xy -0.633613 2.030893)
    (xy -0.939146 1.934399) (xy -1.22961 1.79915) (xy -1.500112 1.627424) (xy -1.746098 1.422115) (xy -1.963425 1.186678)
    (xy -2.148432 0.925079) (xy -2.298003 0.641724) (xy -2.409619 0.341385) (xy -2.481402 0.029122) (xy -2.512141 -0.289808)
    (xy -2.5016 -0.601715) (xy -2.5016 -0.854591))
   (layer "F.Cu") (width 0) (fill solid))
  (fp_poly
   (pts (xy 2.5016 -0.601715) (xy 2.512141 -0.289808) (xy 2.481402 0.029122) (xy 2.409619 0.341385) (xy 2.298003 0.641724)
    (xy 2.148432 0.925079) (xy 1.963425 1.186678) (xy 1.746098 1.422115) (xy 1.500112 1.627424) (xy 1.22961 1.79915) (xy 0.939146 1.934399)
    (xy 0.633613 2.030893) (xy 0.318157 2.087008) (xy 0.002346 2.1016) (xy -0.002347 2.1016) (xy -0.318157 2.087007) (xy -0.633613 2.030893)
    (xy -0.939146 1.934398) (xy -1.22961 1.799149) (xy -1.500112 1.627423) (xy -1.746098 1.422114) (xy -1.963424 1.186677)
    (xy -2.148431 0.925078) (xy -2.298003 0.641723) (xy -2.409619 0.341384) (xy -2.482146 0.025885) (xy -2.50954 -0.853224)
    (xy -2.32514 -0.668824) (xy -2.101909 -0.404578) (xy -1.857026 -0.174874) (xy -1.587231 0.024961) (xy -1.29613 0.192254)
    (xy -0.987628 0.324762) (xy -0.665875 0.4207) (xy -0.335185 0.478783) (xy 0.000001 0.49823) (xy 0.335186 0.478783)
    (xy 0.665876 0.420699) (xy 0.987629 0.324761) (xy 1.296131 0.192254) (xy 1.587233 0.02496) (xy 1.854655 -0.173117) (xy 2.5016 -0.854591))
   (layer "B.Cu") (width 0) (fill solid)))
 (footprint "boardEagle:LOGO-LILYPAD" (layer "B.Cu") (at 148.5011 105.0036 180)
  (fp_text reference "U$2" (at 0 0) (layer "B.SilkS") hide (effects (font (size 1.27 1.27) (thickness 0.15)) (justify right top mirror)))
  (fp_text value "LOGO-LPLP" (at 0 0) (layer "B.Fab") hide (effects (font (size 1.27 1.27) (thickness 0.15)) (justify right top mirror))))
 (gr_circle (center 148.5011 105.0036) (end 158.5011 105.0036) (layer "Edge.Cuts") (width 0.2032) (fill none))
 (segment (start 147.5511 106.0036) (end 147.5011 106.0036) (width 0.4064) (layer "F.Cu") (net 2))
 (segment (start 145.9611 107.5436) (end 144.7011 108.8036) (width 0.254) (layer "F.Cu") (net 2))
 (segment (start 144.7011 108.8036) (end 141.9011 108.8036) (width 0.254) (layer "F.Cu") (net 2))
 (segment (start 145.9611 105.8536) (end 145.9611 107.5436) (width 0.254) (layer "F.Cu") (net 2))
 (segment (start 147.4011 105.8536) (end 145.9611 105.8536) (width 0.254) (layer "F.Cu") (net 2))
 (segment (start 147.5511 106.0036) (end 147.4011 105.8536) (width 0.254) (layer "F.Cu") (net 2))
 (segment (start 147.9501 103.9036) (end 147.7001 104.1536) (width 0.254) (layer "F.Cu") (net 3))
 (segment (start 148.5011 103.9036) (end 148.5011 97.4036) (width 0.254) (layer "F.Cu") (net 3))
 (segment (start 148.5011 103.9036) (end 147.9501 103.9036) (width 0.254) (layer "F.Cu") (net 3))
 (segment (start 147.7001 104.1536) (end 145.9611 104.1536) (width 0.254) (layer "F.Cu") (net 3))
 (segment (start 152.3011 106.0036) (end 155.1011 108.8036) (width 0.254) (layer "F.Cu") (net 1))
 (segment (start 149.4511 106.0036) (end 149.5011 106.0036) (width 0.4064) (layer "F.Cu") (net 1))
 (segment (start 149.5011 106.0036) (end 152.3011 106.0036) (width 0.254) (layer "F.Cu") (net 1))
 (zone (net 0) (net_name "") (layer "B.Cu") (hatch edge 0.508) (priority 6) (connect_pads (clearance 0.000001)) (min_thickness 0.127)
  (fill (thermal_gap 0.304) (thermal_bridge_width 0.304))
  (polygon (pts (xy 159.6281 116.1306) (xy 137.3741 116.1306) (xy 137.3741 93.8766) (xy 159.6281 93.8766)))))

